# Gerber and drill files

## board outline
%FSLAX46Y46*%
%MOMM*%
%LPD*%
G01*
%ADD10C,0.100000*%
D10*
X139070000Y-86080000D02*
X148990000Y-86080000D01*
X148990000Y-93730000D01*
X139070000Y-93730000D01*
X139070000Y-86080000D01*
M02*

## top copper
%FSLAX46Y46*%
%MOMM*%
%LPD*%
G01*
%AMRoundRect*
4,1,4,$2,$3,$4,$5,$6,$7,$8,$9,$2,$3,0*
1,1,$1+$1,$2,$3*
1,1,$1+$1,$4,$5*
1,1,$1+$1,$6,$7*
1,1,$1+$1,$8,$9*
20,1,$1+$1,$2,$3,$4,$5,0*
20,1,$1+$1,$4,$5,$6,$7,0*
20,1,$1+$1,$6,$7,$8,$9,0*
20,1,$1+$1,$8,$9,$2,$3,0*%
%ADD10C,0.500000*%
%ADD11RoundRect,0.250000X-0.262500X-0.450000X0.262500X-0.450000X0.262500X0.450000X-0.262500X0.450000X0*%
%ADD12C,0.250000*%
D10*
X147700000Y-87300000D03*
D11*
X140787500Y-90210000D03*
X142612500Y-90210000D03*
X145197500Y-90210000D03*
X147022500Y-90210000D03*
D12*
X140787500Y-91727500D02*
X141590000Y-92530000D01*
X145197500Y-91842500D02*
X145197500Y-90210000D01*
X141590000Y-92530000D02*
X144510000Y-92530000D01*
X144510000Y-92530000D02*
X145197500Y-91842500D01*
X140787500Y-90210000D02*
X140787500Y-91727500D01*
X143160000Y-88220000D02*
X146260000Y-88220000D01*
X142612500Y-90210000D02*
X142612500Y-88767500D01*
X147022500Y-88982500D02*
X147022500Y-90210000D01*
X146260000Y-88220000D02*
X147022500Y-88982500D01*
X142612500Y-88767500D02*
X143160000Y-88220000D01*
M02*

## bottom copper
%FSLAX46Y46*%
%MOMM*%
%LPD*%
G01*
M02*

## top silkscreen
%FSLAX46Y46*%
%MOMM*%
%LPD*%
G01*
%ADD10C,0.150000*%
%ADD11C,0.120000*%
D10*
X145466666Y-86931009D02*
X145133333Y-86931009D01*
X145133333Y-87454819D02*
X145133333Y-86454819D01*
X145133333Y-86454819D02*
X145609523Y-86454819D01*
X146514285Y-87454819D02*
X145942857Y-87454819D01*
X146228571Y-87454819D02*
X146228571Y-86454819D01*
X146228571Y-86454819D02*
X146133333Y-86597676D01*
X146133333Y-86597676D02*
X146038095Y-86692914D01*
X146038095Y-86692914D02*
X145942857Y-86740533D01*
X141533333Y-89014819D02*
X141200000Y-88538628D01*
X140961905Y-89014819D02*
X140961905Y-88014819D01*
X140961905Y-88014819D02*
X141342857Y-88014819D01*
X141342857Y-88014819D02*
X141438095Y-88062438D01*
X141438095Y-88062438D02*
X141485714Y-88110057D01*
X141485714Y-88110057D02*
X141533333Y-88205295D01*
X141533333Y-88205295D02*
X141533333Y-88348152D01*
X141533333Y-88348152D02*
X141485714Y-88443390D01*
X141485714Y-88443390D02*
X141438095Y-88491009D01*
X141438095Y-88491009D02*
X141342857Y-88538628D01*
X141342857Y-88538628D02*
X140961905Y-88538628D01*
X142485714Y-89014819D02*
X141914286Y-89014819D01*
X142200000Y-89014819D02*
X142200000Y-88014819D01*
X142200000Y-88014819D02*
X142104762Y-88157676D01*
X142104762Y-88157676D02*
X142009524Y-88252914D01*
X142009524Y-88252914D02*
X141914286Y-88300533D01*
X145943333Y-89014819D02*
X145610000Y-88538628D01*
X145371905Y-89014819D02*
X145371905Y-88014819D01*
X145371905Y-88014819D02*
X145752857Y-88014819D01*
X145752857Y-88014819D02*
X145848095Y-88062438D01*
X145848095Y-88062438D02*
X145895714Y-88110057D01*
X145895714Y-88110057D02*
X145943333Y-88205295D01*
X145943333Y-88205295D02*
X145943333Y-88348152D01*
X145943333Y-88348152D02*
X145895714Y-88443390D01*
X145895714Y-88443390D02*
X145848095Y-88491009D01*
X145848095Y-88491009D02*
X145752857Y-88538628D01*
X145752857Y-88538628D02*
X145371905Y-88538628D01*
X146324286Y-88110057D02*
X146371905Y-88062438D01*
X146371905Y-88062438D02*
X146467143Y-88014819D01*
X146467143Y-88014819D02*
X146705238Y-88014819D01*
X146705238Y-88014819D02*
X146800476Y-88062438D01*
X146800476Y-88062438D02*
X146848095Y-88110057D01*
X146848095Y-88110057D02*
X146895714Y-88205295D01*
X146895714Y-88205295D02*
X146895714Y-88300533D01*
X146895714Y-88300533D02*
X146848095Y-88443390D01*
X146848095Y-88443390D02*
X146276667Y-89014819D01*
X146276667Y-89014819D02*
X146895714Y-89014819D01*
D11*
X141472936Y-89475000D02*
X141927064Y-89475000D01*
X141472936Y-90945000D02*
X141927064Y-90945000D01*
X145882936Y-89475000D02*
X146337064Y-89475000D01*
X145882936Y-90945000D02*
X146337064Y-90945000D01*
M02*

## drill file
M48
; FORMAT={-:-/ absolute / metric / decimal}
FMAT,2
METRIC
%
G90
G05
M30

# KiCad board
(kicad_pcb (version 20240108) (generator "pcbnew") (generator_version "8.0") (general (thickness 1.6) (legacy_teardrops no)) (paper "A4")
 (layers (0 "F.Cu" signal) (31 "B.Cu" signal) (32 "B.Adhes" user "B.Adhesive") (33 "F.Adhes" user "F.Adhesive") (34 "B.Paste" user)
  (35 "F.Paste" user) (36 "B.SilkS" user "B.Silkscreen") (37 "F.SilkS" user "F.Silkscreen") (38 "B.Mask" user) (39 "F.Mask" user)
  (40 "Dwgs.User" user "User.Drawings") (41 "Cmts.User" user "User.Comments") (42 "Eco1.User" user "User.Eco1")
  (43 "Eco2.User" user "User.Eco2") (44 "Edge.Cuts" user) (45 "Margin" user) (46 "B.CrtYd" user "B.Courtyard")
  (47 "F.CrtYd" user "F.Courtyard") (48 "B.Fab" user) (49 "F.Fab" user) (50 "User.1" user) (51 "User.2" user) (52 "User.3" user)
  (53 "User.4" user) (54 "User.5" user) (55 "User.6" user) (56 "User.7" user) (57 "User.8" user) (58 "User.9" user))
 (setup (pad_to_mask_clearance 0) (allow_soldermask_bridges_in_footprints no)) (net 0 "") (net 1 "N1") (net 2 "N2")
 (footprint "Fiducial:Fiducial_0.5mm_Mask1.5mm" (layer "F.Cu") (at 147.7 87.3)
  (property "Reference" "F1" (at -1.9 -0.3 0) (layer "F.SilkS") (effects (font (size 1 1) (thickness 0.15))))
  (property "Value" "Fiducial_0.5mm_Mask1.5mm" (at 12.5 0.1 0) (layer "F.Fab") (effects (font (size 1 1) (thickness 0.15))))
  (pad "" smd circle (at 0 0) (size 0.5 0.5) (layers "F.Cu" "F.Mask") (solder_mask_margin 0.5) (clearance 0.5)))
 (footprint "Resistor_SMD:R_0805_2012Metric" (layer "F.Cu") (at 141.7 90.21)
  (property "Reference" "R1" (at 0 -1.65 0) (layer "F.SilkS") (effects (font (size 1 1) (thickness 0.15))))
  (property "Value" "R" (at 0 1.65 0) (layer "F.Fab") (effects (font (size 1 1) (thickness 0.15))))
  (fp_line (start -0.227064 -0.735) (end 0.227064 -0.735) (stroke (width 0.12) (type solid)) (layer "F.SilkS"))
  (fp_line (start -0.227064 0.735) (end 0.227064 0.735) (stroke (width 0.12) (type solid)) (layer "F.SilkS"))
  (pad "1" smd roundrect (at -0.9125 0) (size 1.025 1.4) (layers "F.Cu" "F.Paste" "F.Mask") (roundrect_rratio 0.243902) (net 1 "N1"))
  (pad "2" smd roundrect (at 0.9125 0) (size 1.025 1.4) (layers "F.Cu" "F.Paste" "F.Mask") (roundrect_rratio 0.243902) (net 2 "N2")))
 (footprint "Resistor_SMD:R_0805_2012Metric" (layer "F.Cu") (at 146.11 90.21)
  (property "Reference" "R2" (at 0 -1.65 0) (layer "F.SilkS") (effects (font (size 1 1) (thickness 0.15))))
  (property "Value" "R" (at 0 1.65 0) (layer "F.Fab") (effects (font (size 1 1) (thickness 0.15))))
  (fp_line (start -0.227064 -0.735) (end 0.227064 -0.735) (stroke (width 0.12) (type solid)) (layer "F.SilkS"))
  (fp_line (start -0.227064 0.735) (end 0.227064 0.735) (stroke (width 0.12) (type solid)) (layer "F.SilkS"))
  (pad "1" smd roundrect (at -0.9125 0) (size 1.025 1.4) (layers "F.Cu" "F.Paste" "F.Mask") (roundrect_rratio 0.243902) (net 1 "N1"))
  (pad "2" smd roundrect (at 0.9125 0) (size 1.025 1.4) (layers "F.Cu" "F.Paste" "F.Mask") (roundrect_rratio 0.243902) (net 2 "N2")))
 (gr_rect (start 139.07 86.08) (end 148.99 93.73) (stroke (width 0.1) (type solid)) (fill none) (layer "Edge.Cuts"))
 (segment (start 140.7875 91.7275) (end 141.59 92.53) (width 0.25) (layer "F.Cu") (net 1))
 (segment (start 145.1975 91.8425) (end 145.1975 90.21) (width 0.25) (layer "F.Cu") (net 1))
 (segment (start 141.59 92.53) (end 144.51 92.53) (width 0.25) (layer "F.Cu") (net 1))
 (segment (start 144.51 92.53) (end 145.1975 91.8425) (width 0.25) (layer "F.Cu") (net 1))
 (segment (start 140.7875 90.21) (end 140.7875 91.7275) (width 0.25) (layer "F.Cu") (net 1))
 (segment (start 143.16 88.22) (end 146.26 88.22) (width 0.25) (layer "F.Cu") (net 2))
 (segment (start 142.6125 90.21) (end 142.6125 88.7675) (width 0.25) (layer "F.Cu") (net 2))
 (segment (start 147.0225 88.9825) (end 147.0225 90.21) (width 0.25) (layer "F.Cu") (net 2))
 (segment (start 146.26 88.22) (end 147.0225 88.9825) (width 0.25) (layer "F.Cu") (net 2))
 (segment (start 142.6125 88.7675) (end 143.16 88.22) (width 0.25) (layer "F.Cu") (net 2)))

